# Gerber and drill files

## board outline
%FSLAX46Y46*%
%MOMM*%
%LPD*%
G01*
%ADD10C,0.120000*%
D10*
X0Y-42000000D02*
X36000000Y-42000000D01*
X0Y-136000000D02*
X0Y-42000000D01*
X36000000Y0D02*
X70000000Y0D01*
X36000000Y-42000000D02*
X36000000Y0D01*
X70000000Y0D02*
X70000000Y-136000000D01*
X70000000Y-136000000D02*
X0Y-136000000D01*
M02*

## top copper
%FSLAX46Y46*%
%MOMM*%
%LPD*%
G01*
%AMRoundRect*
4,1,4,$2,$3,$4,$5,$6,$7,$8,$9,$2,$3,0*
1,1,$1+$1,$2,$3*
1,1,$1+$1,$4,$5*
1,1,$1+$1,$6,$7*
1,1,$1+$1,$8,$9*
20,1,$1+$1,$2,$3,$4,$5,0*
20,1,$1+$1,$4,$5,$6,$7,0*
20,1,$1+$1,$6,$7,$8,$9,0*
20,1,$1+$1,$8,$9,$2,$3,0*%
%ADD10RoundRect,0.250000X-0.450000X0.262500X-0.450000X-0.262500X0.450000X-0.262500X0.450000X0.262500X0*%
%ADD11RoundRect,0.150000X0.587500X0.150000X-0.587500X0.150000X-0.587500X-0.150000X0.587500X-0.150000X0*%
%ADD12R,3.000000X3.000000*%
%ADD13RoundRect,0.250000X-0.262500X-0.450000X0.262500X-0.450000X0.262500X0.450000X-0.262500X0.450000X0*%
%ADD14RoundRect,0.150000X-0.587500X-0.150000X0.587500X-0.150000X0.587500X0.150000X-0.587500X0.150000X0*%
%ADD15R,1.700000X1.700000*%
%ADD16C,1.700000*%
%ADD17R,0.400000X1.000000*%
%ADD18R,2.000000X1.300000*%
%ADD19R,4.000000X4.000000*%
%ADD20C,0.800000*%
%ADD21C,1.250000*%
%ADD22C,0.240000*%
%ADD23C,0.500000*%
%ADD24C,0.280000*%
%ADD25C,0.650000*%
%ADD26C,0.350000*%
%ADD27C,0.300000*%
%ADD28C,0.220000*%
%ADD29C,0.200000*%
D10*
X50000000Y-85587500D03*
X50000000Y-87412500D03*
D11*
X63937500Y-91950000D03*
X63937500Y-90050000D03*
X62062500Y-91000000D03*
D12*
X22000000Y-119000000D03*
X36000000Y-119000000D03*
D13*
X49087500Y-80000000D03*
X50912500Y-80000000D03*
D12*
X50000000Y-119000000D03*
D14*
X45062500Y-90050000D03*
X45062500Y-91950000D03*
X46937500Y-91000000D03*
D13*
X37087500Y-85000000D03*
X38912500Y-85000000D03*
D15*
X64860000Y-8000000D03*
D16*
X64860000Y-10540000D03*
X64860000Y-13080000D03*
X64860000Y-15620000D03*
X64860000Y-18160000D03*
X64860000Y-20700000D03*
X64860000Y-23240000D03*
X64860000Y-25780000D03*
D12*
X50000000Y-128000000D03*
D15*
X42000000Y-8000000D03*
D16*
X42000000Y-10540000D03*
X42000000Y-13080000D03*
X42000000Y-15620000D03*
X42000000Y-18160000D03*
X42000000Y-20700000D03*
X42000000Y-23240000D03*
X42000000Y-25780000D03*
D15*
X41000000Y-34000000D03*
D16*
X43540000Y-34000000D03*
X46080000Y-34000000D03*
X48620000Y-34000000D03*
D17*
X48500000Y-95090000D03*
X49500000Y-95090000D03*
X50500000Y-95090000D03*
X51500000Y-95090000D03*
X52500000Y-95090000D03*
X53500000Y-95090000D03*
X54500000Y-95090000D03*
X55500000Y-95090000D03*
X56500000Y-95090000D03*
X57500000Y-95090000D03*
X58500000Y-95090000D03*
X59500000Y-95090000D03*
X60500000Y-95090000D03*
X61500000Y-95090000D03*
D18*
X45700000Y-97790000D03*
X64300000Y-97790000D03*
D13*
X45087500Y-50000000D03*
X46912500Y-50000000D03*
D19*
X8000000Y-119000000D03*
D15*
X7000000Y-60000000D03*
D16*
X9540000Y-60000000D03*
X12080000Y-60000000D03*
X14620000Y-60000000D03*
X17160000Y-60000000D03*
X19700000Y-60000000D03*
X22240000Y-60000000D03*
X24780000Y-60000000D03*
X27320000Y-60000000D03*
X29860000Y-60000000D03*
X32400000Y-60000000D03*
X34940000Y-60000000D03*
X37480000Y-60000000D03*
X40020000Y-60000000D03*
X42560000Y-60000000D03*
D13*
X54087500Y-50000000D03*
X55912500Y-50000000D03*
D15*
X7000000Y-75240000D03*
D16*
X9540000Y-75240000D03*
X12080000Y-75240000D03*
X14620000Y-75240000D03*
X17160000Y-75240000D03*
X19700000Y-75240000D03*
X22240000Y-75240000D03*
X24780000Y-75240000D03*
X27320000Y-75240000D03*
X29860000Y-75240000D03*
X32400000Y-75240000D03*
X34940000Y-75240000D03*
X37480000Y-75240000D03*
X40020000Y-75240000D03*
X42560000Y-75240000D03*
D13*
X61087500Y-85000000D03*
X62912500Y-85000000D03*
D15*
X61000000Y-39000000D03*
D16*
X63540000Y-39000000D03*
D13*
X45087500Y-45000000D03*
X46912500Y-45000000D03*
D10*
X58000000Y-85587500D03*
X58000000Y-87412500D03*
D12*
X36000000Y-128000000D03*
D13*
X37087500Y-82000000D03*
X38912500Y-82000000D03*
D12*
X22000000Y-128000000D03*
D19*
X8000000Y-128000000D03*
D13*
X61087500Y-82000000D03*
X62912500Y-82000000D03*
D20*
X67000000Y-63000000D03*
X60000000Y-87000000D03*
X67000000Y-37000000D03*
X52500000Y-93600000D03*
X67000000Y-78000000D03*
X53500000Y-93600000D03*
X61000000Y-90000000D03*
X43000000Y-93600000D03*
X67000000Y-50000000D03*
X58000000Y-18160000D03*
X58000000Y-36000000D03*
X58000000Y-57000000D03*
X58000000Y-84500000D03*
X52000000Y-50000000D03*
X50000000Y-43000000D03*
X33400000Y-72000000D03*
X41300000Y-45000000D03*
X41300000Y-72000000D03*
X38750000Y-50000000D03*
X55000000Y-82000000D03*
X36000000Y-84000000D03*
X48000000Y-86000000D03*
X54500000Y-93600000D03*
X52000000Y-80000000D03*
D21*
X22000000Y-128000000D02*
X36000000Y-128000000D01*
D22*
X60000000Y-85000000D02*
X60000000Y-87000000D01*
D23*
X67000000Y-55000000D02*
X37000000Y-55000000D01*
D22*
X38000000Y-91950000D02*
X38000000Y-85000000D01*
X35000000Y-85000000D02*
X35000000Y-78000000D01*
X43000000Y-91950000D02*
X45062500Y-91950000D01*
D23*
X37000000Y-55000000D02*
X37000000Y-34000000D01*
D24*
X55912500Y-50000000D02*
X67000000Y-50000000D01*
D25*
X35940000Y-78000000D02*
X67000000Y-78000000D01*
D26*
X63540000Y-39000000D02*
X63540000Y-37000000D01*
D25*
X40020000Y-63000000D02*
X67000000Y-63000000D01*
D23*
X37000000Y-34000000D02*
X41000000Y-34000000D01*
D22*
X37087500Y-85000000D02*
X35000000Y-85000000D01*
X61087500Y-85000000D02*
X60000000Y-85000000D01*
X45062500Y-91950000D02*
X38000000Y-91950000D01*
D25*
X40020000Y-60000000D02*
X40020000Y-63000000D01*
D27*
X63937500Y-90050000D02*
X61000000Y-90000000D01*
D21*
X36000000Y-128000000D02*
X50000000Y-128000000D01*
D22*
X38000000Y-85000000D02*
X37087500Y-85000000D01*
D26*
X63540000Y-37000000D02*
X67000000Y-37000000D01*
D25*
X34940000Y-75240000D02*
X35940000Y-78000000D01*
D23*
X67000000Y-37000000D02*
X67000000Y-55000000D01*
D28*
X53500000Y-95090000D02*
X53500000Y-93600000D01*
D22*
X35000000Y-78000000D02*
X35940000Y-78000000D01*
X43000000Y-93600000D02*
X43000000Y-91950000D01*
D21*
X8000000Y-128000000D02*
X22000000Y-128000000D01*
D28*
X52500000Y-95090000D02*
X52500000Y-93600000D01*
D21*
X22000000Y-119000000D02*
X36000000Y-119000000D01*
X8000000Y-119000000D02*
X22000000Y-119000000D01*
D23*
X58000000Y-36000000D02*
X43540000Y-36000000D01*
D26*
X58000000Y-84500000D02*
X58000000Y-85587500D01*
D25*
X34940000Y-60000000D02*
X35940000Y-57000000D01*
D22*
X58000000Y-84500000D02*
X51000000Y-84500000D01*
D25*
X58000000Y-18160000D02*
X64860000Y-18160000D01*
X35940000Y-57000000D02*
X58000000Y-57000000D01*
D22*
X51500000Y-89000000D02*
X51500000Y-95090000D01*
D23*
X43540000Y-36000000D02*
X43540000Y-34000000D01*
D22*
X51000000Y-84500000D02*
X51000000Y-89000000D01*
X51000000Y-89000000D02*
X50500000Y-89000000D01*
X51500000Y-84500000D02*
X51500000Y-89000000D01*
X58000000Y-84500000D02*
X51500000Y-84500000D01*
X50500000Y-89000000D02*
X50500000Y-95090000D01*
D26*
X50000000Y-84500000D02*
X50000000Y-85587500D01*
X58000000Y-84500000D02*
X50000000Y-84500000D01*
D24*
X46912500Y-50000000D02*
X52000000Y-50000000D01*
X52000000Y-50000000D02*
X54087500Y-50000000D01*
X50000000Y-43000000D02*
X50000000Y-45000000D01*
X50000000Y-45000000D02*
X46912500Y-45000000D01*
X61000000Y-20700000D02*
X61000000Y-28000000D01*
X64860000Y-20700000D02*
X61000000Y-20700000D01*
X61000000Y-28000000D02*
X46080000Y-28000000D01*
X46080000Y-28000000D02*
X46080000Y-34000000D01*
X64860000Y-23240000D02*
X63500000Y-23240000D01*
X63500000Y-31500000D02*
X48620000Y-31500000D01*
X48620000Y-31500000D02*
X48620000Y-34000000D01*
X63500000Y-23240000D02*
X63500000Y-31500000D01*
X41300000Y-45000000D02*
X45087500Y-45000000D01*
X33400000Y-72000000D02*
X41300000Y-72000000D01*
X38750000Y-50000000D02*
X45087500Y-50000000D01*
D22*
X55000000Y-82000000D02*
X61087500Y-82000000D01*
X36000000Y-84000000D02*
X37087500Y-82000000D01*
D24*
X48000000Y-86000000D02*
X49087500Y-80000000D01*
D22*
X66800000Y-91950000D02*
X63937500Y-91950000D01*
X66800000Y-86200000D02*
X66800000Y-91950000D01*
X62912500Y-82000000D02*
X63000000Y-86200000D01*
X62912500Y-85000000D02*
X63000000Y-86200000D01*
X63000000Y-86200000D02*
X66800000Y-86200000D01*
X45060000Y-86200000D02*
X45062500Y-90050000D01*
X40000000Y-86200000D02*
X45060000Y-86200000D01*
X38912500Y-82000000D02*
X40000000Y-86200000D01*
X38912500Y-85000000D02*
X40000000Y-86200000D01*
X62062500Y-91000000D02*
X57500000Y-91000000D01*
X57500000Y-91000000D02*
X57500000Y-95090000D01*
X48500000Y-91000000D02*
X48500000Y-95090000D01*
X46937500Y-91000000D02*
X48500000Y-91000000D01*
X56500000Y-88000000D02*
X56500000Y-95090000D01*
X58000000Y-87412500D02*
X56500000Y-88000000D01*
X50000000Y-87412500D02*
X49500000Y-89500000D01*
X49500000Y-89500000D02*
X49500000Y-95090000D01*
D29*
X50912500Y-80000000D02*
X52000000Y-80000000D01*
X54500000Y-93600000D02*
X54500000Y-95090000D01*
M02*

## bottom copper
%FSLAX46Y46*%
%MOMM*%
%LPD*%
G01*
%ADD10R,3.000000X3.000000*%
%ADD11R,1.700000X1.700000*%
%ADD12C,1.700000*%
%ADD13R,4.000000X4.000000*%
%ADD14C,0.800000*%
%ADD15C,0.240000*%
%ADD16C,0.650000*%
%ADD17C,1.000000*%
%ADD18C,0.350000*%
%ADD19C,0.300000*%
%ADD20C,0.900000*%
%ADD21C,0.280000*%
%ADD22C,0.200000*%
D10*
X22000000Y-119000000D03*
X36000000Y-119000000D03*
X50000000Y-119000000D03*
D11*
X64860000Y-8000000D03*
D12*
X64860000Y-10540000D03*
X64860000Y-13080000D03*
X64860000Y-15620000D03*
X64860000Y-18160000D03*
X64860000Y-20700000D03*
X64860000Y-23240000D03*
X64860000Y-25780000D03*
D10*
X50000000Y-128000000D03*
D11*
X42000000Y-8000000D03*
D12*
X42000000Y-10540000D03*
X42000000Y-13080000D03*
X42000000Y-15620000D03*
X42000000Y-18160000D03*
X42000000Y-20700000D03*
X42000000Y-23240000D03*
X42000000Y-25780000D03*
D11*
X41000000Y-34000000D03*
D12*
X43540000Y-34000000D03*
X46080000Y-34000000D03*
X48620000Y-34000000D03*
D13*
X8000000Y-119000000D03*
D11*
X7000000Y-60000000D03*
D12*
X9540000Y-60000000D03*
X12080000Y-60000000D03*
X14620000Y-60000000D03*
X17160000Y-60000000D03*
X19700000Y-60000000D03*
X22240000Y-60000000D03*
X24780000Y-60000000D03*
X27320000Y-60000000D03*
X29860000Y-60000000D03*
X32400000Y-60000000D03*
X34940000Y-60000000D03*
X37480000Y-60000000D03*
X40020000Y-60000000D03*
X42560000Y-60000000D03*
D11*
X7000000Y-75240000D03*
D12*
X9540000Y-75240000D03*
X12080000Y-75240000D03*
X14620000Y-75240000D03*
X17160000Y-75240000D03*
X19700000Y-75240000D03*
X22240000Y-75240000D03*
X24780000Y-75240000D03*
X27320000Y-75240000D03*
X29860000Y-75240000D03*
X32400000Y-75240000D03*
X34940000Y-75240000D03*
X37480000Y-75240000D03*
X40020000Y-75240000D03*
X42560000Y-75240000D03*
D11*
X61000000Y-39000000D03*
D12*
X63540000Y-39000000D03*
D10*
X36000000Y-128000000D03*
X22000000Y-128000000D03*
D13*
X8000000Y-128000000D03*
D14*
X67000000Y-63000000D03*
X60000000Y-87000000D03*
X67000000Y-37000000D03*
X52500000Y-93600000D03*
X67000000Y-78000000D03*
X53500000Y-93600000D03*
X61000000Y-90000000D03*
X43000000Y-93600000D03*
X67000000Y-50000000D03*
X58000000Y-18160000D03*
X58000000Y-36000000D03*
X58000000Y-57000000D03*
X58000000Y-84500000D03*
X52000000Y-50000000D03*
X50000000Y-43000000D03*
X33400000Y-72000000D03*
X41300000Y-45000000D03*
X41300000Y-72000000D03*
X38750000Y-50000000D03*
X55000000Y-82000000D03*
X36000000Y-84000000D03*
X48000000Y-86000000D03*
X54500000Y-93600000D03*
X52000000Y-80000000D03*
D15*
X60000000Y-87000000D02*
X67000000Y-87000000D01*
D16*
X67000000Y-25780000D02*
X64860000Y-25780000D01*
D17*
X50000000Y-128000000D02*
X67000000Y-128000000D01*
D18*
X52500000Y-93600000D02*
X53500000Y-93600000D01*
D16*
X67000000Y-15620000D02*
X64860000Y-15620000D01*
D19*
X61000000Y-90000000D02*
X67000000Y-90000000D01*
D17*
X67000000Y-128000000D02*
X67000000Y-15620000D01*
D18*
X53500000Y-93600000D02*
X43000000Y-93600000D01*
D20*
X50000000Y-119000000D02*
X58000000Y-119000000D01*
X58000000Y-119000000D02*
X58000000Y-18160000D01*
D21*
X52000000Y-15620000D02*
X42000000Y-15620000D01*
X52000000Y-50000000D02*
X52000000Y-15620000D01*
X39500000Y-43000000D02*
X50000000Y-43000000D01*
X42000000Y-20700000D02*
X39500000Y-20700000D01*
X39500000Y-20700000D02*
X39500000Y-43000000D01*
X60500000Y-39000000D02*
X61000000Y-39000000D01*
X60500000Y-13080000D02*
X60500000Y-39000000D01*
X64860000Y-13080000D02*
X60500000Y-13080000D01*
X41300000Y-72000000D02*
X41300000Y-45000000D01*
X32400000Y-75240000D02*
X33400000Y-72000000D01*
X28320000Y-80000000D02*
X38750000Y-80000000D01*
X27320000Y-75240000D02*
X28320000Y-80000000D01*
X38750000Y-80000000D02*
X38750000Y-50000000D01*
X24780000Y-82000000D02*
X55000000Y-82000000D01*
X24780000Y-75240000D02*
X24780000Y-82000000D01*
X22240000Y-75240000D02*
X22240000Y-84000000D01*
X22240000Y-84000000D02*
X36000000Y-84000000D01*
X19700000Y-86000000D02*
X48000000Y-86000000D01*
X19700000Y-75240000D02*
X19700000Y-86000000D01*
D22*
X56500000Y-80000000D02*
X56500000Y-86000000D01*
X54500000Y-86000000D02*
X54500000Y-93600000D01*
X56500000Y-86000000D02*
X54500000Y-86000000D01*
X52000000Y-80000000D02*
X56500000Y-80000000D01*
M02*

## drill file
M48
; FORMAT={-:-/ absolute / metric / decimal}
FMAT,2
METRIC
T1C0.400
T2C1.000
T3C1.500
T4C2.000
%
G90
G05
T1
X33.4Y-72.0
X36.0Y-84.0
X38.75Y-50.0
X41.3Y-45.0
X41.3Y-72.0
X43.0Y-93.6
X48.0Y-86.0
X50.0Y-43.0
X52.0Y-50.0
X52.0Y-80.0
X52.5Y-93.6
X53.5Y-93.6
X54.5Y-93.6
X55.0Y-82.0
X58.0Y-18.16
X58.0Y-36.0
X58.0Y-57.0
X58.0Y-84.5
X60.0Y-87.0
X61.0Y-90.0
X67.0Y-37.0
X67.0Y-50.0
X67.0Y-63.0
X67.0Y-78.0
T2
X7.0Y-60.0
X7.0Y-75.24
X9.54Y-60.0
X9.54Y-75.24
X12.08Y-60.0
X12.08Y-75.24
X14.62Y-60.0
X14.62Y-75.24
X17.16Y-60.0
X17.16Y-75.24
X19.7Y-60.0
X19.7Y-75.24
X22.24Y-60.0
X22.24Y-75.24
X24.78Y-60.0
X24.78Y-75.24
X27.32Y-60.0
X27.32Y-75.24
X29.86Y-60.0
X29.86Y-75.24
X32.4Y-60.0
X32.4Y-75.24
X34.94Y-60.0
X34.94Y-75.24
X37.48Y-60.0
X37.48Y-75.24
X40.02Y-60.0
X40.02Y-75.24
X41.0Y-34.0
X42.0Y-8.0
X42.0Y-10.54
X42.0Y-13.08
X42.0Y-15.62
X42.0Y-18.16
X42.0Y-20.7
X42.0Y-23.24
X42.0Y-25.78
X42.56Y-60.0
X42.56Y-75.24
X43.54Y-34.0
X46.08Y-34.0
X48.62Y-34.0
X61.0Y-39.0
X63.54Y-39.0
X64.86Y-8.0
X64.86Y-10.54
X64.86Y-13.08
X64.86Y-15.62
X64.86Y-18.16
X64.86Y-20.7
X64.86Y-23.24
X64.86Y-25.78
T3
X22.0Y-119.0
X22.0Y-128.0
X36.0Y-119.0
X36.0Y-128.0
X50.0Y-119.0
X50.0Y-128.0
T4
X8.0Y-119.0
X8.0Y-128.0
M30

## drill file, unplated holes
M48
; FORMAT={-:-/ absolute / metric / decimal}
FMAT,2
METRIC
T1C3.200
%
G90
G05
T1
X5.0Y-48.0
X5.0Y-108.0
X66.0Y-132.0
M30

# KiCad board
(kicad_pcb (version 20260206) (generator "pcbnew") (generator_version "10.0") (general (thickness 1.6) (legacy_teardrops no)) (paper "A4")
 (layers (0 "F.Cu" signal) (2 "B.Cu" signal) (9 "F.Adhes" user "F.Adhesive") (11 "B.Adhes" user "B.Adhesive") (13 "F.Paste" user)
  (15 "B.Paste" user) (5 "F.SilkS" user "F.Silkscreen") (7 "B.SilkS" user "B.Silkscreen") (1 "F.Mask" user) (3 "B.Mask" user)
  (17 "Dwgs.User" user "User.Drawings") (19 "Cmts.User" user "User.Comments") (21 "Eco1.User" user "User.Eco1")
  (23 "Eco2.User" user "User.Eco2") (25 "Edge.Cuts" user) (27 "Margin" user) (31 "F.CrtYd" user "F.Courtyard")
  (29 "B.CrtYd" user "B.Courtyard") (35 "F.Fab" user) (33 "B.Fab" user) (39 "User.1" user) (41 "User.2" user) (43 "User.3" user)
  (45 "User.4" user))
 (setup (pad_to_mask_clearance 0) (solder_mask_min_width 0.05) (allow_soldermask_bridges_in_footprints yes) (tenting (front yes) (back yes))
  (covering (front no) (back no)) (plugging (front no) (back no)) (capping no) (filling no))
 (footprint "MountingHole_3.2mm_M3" (layer "F.Cu") (at 5 48)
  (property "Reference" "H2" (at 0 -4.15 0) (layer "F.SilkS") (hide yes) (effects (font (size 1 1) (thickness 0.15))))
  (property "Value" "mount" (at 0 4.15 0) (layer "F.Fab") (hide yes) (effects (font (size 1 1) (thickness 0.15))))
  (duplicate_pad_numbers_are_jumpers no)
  (pad "" np_thru_hole circle (at 0 0) (size 3.2 3.2) (drill 3.2) (layers "*.Cu" "*.Mask")))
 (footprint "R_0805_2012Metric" (layer "F.Cu") (at 50 86.5 -90)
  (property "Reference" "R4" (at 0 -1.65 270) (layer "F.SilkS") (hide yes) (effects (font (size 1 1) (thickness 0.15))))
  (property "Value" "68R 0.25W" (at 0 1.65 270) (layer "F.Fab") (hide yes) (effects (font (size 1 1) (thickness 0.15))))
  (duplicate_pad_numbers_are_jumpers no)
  (pad "1" smd roundrect (at -0.9125 0 270) (size 1.025 1.4) (layers "F.Cu" "F.Mask" "F.Paste") (roundrect_rratio 0.243902) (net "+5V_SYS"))
  (pad "2" smd roundrect (at 0.9125 0 270) (size 1.025 1.4) (layers "F.Cu" "F.Mask" "F.Paste") (roundrect_rratio 0.243902) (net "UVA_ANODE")))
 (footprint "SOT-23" (layer "F.Cu") (at 63 91 180)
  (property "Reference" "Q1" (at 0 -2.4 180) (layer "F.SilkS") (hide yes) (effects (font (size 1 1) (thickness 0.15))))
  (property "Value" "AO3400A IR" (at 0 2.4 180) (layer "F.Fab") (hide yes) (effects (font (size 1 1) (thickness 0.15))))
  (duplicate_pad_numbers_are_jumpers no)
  (pad "1" smd roundrect (at -0.9375 -0.95 180) (size 1.475 0.6) (layers "F.Cu" "F.Mask" "F.Paste") (roundrect_rratio 0.25) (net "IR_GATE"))
  (pad "2" smd roundrect (at -0.9375 0.95 180) (size 1.475 0.6) (layers "F.Cu" "F.Mask" "F.Paste") (roundrect_rratio 0.25) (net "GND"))
  (pad "3" smd roundrect (at 0.9375 0 180) (size 1.475 0.6) (layers "F.Cu" "F.Mask" "F.Paste") (roundrect_rratio 0.25) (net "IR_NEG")))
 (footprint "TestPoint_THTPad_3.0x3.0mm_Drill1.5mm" (layer "F.Cu") (at 22 119)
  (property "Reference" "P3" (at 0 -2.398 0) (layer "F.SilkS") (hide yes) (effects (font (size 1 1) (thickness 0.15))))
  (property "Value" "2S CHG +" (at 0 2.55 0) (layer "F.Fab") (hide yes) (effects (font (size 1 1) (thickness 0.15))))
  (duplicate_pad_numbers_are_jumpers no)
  (pad "1" thru_hole rect (at 0 0) (size 3 3) (drill 1.5) (layers "*.Cu" "*.Mask") (remove_unused_layers no) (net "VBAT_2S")))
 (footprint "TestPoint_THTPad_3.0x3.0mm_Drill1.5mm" (layer "F.Cu") (at 36 119)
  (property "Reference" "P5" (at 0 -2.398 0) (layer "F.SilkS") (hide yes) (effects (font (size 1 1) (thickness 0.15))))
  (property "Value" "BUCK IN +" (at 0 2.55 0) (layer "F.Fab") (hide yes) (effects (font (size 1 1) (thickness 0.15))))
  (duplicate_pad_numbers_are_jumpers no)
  (pad "1" thru_hole rect (at 0 0) (size 3 3) (drill 1.5) (layers "*.Cu" "*.Mask") (remove_unused_layers no) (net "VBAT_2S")))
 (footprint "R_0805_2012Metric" (layer "F.Cu") (at 50 80)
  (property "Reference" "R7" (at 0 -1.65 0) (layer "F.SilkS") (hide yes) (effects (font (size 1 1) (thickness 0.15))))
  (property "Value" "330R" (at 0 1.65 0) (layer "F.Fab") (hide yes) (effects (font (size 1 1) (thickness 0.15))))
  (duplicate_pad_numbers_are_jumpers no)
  (pad "1" smd roundrect (at -0.9125 0) (size 1.025 1.4) (layers "F.Cu" "F.Mask" "F.Paste") (roundrect_rratio 0.243902)
   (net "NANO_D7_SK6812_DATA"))
  (pad "2" smd roundrect (at 0.9125 0) (size 1.025 1.4) (layers "F.Cu" "F.Mask" "F.Paste") (roundrect_rratio 0.243902) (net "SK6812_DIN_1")))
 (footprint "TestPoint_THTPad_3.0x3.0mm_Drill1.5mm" (layer "F.Cu") (at 50 119)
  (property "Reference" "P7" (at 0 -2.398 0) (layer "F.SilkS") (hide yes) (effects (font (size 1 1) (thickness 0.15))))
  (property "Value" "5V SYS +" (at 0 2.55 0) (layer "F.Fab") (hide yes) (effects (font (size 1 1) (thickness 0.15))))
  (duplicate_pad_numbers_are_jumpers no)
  (pad "1" thru_hole rect (at 0 0) (size 3 3) (drill 1.5) (layers "*.Cu" "*.Mask") (remove_unused_layers no) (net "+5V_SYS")))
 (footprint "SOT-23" (layer "F.Cu") (at 46 91)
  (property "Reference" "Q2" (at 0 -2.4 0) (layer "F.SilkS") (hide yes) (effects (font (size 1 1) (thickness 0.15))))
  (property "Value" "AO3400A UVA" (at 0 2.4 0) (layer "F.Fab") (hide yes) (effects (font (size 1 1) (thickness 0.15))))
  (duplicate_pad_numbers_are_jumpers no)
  (pad "1" smd roundrect (at -0.9375 -0.95) (size 1.475 0.6) (layers "F.Cu" "F.Mask" "F.Paste") (roundrect_rratio 0.25) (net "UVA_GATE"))
  (pad "2" smd roundrect (at -0.9375 0.95) (size 1.475 0.6) (layers "F.Cu" "F.Mask" "F.Paste") (roundrect_rratio 0.25) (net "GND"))
  (pad "3" smd roundrect (at 0.9375 0) (size 1.475 0.6) (layers "F.Cu" "F.Mask" "F.Paste") (roundrect_rratio 0.25) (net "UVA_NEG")))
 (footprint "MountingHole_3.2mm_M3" (layer "F.Cu") (at 66 132)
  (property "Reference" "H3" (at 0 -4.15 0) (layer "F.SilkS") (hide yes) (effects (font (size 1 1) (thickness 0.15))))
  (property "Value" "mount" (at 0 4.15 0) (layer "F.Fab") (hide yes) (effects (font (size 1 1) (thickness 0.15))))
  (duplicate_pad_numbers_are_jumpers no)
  (pad "" np_thru_hole circle (at 0 0) (size 3.2 3.2) (drill 3.2) (layers "*.Cu" "*.Mask")))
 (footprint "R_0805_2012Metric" (layer "F.Cu") (at 38 85)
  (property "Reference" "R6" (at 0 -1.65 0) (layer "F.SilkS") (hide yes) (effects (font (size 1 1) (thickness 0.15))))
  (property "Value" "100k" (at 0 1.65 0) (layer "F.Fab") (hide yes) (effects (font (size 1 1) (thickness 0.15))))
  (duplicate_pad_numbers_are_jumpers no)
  (pad "1" smd roundrect (at -0.9125 0) (size 1.025 1.4) (layers "F.Cu" "F.Mask" "F.Paste") (roundrect_rratio 0.243902) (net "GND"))
  (pad "2" smd roundrect (at 0.9125 0) (size 1.025 1.4) (layers "F.Cu" "F.Mask" "F.Paste") (roundrect_rratio 0.243902) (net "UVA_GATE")))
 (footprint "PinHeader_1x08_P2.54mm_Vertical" (layer "F.Cu") (at 64.86 8)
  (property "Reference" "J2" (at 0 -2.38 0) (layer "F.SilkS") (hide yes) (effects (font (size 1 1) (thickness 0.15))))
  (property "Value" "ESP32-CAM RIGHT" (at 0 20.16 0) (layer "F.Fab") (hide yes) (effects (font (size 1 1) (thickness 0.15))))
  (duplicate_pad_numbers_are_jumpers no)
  (pad "1" thru_hole rect (at 0 0) (size 1.7 1.7) (drill 1) (layers "*.Cu" "*.Mask") (remove_unused_layers no))
  (pad "2" thru_hole circle (at 0 2.54) (size 1.7 1.7) (drill 1) (layers "*.Cu" "*.Mask") (remove_unused_layers no))
  (pad "3" thru_hole circle (at 0 5.08) (size 1.7 1.7) (drill 1) (layers "*.Cu" "*.Mask") (remove_unused_layers no) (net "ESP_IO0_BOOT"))
  (pad "4" thru_hole circle (at 0 7.62) (size 1.7 1.7) (drill 1) (layers "*.Cu" "*.Mask") (remove_unused_layers no) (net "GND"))
  (pad "5" thru_hole circle (at 0 10.16) (size 1.7 1.7) (drill 1) (layers "*.Cu" "*.Mask") (remove_unused_layers no) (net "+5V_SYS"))
  (pad "6" thru_hole circle (at 0 12.7) (size 1.7 1.7) (drill 1) (layers "*.Cu" "*.Mask") (remove_unused_layers no) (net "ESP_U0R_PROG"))
  (pad "7" thru_hole circle (at 0 15.24) (size 1.7 1.7) (drill 1) (layers "*.Cu" "*.Mask") (remove_unused_layers no) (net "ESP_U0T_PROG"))
  (pad "8" thru_hole circle (at 0 17.78) (size 1.7 1.7) (drill 1) (layers "*.Cu" "*.Mask") (remove_unused_layers no) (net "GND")))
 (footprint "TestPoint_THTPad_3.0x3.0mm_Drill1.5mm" (layer "F.Cu") (at 50 128)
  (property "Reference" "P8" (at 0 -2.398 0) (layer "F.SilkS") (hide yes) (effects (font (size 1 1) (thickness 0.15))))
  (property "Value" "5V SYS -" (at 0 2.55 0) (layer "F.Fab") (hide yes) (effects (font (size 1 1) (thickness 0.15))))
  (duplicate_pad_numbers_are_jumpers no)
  (pad "1" thru_hole rect (at 0 0) (size 3 3) (drill 1.5) (layers "*.Cu" "*.Mask") (remove_unused_layers no) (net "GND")))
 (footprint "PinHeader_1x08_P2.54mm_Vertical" (layer "F.Cu") (at 42 8)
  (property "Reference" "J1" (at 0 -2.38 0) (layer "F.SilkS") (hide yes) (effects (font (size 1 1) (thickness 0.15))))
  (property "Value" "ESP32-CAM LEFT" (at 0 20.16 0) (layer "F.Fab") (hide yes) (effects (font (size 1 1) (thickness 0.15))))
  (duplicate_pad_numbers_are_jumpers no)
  (pad "1" thru_hole rect (at 0 0) (size 1.7 1.7) (drill 1) (layers "*.Cu" "*.Mask") (remove_unused_layers no))
  (pad "2" thru_hole circle (at 0 2.54) (size 1.7 1.7) (drill 1) (layers "*.Cu" "*.Mask") (remove_unused_layers no))
  (pad "3" thru_hole circle (at 0 5.08) (size 1.7 1.7) (drill 1) (layers "*.Cu" "*.Mask") (remove_unused_layers no))
  (pad "4" thru_hole circle (at 0 7.62) (size 1.7 1.7) (drill 1) (layers "*.Cu" "*.Mask") (remove_unused_layers no) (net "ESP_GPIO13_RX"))
  (pad "5" thru_hole circle (at 0 10.16) (size 1.7 1.7) (drill 1) (layers "*.Cu" "*.Mask") (remove_unused_layers no))
  (pad "6" thru_hole circle (at 0 12.7) (size 1.7 1.7) (drill 1) (layers "*.Cu" "*.Mask") (remove_unused_layers no) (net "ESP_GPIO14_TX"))
  (pad "7" thru_hole circle (at 0 15.24) (size 1.7 1.7) (drill 1) (layers "*.Cu" "*.Mask") (remove_unused_layers no))
  (pad "8" thru_hole circle (at 0 17.78) (size 1.7 1.7) (drill 1) (layers "*.Cu" "*.Mask") (remove_unused_layers no)))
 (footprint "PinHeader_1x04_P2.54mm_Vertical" (layer "F.Cu") (at 41 34 90)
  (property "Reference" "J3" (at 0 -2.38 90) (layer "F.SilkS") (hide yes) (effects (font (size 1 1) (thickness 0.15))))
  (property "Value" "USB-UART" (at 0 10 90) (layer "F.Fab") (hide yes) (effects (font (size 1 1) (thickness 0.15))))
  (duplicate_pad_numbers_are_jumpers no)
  (pad "1" thru_hole rect (at 0 0 90) (size 1.7 1.7) (drill 1) (layers "*.Cu" "*.Mask") (remove_unused_layers no) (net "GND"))
  (pad "2" thru_hole circle (at 0 2.54 90) (size 1.7 1.7) (drill 1) (layers "*.Cu" "*.Mask") (remove_unused_layers no) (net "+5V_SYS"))
  (pad "3" thru_hole circle (at 0 5.08 90) (size 1.7 1.7) (drill 1) (layers "*.Cu" "*.Mask") (remove_unused_layers no) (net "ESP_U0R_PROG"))
  (pad "4" thru_hole circle (at 0 7.62 90) (size 1.7 1.7) (drill 1) (layers "*.Cu" "*.Mask") (remove_unused_layers no) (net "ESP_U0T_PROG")))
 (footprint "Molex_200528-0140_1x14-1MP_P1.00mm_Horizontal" (layer "F.Cu") (at 55 96)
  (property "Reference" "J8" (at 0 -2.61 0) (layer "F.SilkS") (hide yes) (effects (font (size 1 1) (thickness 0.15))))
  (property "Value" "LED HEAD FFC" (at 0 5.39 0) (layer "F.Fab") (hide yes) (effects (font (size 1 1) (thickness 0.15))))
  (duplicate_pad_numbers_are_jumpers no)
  (pad "1" smd rect (at -6.5 -0.91) (size 0.4 1) (layers "F.Cu" "F.Mask" "F.Paste") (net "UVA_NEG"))
  (pad "2" smd rect (at -5.5 -0.91) (size 0.4 1) (layers "F.Cu" "F.Mask" "F.Paste") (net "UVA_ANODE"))
  (pad "3" smd rect (at -4.5 -0.91) (size 0.4 1) (layers "F.Cu" "F.Mask" "F.Paste") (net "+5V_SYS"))
  (pad "4" smd rect (at -3.5 -0.91) (size 0.4 1) (layers "F.Cu" "F.Mask" "F.Paste") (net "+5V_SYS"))
  (pad "5" smd rect (at -2.5 -0.91) (size 0.4 1) (layers "F.Cu" "F.Mask" "F.Paste") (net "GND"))
  (pad "6" smd rect (at -1.5 -0.91) (size 0.4 1) (layers "F.Cu" "F.Mask" "F.Paste") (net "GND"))
  (pad "7" smd rect (at -0.5 -0.91) (size 0.4 1) (layers "F.Cu" "F.Mask" "F.Paste") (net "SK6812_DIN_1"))
  (pad "8" smd rect (at 0.5 -0.91) (size 0.4 1) (layers "F.Cu" "F.Mask" "F.Paste"))
  (pad "9" smd rect (at 1.5 -0.91) (size 0.4 1) (layers "F.Cu" "F.Mask" "F.Paste") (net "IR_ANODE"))
  (pad "10" smd rect (at 2.5 -0.91) (size 0.4 1) (layers "F.Cu" "F.Mask" "F.Paste") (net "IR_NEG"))
  (pad "11" smd rect (at 3.5 -0.91) (size 0.4 1) (layers "F.Cu" "F.Mask" "F.Paste"))
  (pad "12" smd rect (at 4.5 -0.91) (size 0.4 1) (layers "F.Cu" "F.Mask" "F.Paste"))
  (pad "13" smd rect (at 5.5 -0.91) (size 0.4 1) (layers "F.Cu" "F.Mask" "F.Paste"))
  (pad "14" smd rect (at 6.5 -0.91) (size 0.4 1) (layers "F.Cu" "F.Mask" "F.Paste"))
  (pad "MP" smd rect (at -9.3 1.79) (size 2 1.3) (layers "F.Cu" "F.Mask" "F.Paste"))
  (pad "MP" smd rect (at 9.3 1.79) (size 2 1.3) (layers "F.Cu" "F.Mask" "F.Paste")))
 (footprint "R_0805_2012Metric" (layer "F.Cu") (at 46 50)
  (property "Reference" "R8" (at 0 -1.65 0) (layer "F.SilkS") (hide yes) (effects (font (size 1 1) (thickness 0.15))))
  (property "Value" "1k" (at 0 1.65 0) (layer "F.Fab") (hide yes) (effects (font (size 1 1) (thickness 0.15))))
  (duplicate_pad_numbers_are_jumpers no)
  (pad "1" smd roundrect (at -0.9125 0) (size 1.025 1.4) (layers "F.Cu" "F.Mask" "F.Paste") (roundrect_rratio 0.243902) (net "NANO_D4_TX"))
  (pad "2" smd roundrect (at 0.9125 0) (size 1.025 1.4) (layers "F.Cu" "F.Mask" "F.Paste") (roundrect_rratio 0.243902) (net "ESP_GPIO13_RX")))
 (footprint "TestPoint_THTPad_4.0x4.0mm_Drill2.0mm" (layer "F.Cu") (at 8 119)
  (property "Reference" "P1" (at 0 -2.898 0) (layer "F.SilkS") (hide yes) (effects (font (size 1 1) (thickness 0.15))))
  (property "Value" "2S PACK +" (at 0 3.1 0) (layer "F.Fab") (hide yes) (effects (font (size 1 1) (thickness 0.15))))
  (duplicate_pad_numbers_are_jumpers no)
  (pad "1" thru_hole rect (at 0 0) (size 4 4) (drill 2) (layers "*.Cu" "*.Mask") (remove_unused_layers no) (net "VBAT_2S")))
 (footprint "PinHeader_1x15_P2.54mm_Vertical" (layer "F.Cu") (at 7 60 90)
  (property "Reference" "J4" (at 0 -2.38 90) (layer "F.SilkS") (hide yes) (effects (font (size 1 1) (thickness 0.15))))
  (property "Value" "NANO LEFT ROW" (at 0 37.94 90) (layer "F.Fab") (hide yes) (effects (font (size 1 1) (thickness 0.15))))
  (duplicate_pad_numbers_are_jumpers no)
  (pad "1" thru_hole rect (at 0 0 90) (size 1.7 1.7) (drill 1) (layers "*.Cu" "*.Mask") (remove_unused_layers no))
  (pad "2" thru_hole circle (at 0 2.54 90) (size 1.7 1.7) (drill 1) (layers "*.Cu" "*.Mask") (remove_unused_layers no))
  (pad "3" thru_hole circle (at 0 5.08 90) (size 1.7 1.7) (drill 1) (layers "*.Cu" "*.Mask") (remove_unused_layers no))
  (pad "4" thru_hole circle (at 0 7.62 90) (size 1.7 1.7) (drill 1) (layers "*.Cu" "*.Mask") (remove_unused_layers no))
  (pad "5" thru_hole circle (at 0 10.16 90) (size 1.7 1.7) (drill 1) (layers "*.Cu" "*.Mask") (remove_unused_layers no))
  (pad "6" thru_hole circle (at 0 12.7 90) (size 1.7 1.7) (drill 1) (layers "*.Cu" "*.Mask") (remove_unused_layers no))
  (pad "7" thru_hole circle (at 0 15.24 90) (size 1.7 1.7) (drill 1) (layers "*.Cu" "*.Mask") (remove_unused_layers no))
  (pad "8" thru_hole circle (at 0 17.78 90) (size 1.7 1.7) (drill 1) (layers "*.Cu" "*.Mask") (remove_unused_layers no))
  (pad "9" thru_hole circle (at 0 20.32 90) (size 1.7 1.7) (drill 1) (layers "*.Cu" "*.Mask") (remove_unused_layers no))
  (pad "10" thru_hole circle (at 0 22.86 90) (size 1.7 1.7) (drill 1) (layers "*.Cu" "*.Mask") (remove_unused_layers no))
  (pad "11" thru_hole circle (at 0 25.4 90) (size 1.7 1.7) (drill 1) (layers "*.Cu" "*.Mask") (remove_unused_layers no))
  (pad "12" thru_hole circle (at 0 27.94 90) (size 1.7 1.7) (drill 1) (layers "*.Cu" "*.Mask") (remove_unused_layers no) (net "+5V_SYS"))
  (pad "13" thru_hole circle (at 0 30.48 90) (size 1.7 1.7) (drill 1) (layers "*.Cu" "*.Mask") (remove_unused_layers no))
  (pad "14" thru_hole circle (at 0 33.02 90) (size 1.7 1.7) (drill 1) (layers "*.Cu" "*.Mask") (remove_unused_layers no) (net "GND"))
  (pad "15" thru_hole circle (at 0 35.56 90) (size 1.7 1.7) (drill 1) (layers "*.Cu" "*.Mask") (remove_unused_layers no)))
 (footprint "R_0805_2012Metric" (layer "F.Cu") (at 55 50)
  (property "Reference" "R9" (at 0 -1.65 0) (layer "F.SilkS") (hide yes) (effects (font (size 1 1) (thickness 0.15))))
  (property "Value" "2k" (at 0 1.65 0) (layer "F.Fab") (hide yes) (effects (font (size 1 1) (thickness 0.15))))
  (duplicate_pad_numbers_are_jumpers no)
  (pad "1" smd roundrect (at -0.9125 0) (size 1.025 1.4) (layers "F.Cu" "F.Mask" "F.Paste") (roundrect_rratio 0.243902)
   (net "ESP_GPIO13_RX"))
  (pad "2" smd roundrect (at 0.9125 0) (size 1.025 1.4) (layers "F.Cu" "F.Mask" "F.Paste") (roundrect_rratio 0.243902) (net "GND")))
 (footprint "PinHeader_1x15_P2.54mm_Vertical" (layer "F.Cu") (at 7 75.24 90)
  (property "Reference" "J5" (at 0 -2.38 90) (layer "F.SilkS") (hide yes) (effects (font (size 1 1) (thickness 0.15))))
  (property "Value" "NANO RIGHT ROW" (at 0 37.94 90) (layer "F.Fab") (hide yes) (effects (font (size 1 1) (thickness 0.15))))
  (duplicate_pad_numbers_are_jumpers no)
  (pad "1" thru_hole rect (at 0 0 90) (size 1.7 1.7) (drill 1) (layers "*.Cu" "*.Mask") (remove_unused_layers no))
  (pad "2" thru_hole circle (at 0 2.54 90) (size 1.7 1.7) (drill 1) (layers "*.Cu" "*.Mask") (remove_unused_layers no))
  (pad "3" thru_hole circle (at 0 5.08 90) (size 1.7 1.7) (drill 1) (layers "*.Cu" "*.Mask") (remove_unused_layers no))
  (pad "4" thru_hole circle (at 0 7.62 90) (size 1.7 1.7) (drill 1) (layers "*.Cu" "*.Mask") (remove_unused_layers no))
  (pad "5" thru_hole circle (at 0 10.16 90) (size 1.7 1.7) (drill 1) (layers "*.Cu" "*.Mask") (remove_unused_layers no)
   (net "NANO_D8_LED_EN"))
  (pad "6" thru_hole circle (at 0 12.7 90) (size 1.7 1.7) (drill 1) (layers "*.Cu" "*.Mask") (remove_unused_layers no)
   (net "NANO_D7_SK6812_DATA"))
  (pad "7" thru_hole circle (at 0 15.24 90) (size 1.7 1.7) (drill 1) (layers "*.Cu" "*.Mask") (remove_unused_layers no)
   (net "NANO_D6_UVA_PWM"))
  (pad "8" thru_hole circle (at 0 17.78 90) (size 1.7 1.7) (drill 1) (layers "*.Cu" "*.Mask") (remove_unused_layers no)
   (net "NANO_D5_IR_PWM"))
  (pad "9" thru_hole circle (at 0 20.32 90) (size 1.7 1.7) (drill 1) (layers "*.Cu" "*.Mask") (remove_unused_layers no) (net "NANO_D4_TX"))
  (pad "10" thru_hole circle (at 0 22.86 90) (size 1.7 1.7) (drill 1) (layers "*.Cu" "*.Mask") (remove_unused_layers no))
  (pad "11" thru_hole circle (at 0 25.4 90) (size 1.7 1.7) (drill 1) (layers "*.Cu" "*.Mask") (remove_unused_layers no) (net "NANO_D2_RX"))
  (pad "12" thru_hole circle (at 0 27.94 90) (size 1.7 1.7) (drill 1) (layers "*.Cu" "*.Mask") (remove_unused_layers no) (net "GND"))
  (pad "13" thru_hole circle (at 0 30.48 90) (size 1.7 1.7) (drill 1) (layers "*.Cu" "*.Mask") (remove_unused_layers no))
  (pad "14" thru_hole circle (at 0 33.02 90) (size 1.7 1.7) (drill 1) (layers "*.Cu" "*.Mask") (remove_unused_layers no))
  (pad "15" thru_hole circle (at 0 35.56 90) (size 1.7 1.7) (drill 1) (layers "*.Cu" "*.Mask") (remove_unused_layers no)))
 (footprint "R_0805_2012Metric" (layer "F.Cu") (at 62 85)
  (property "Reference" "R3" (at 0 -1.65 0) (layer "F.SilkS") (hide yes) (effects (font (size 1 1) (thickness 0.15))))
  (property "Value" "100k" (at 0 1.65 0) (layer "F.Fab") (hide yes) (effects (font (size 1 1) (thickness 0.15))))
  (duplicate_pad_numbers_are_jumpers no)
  (pad "1" smd roundrect (at -0.9125 0) (size 1.025 1.4) (layers "F.Cu" "F.Mask" "F.Paste") (roundrect_rratio 0.243902) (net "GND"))
  (pad "2" smd roundrect (at 0.9125 0) (size 1.025 1.4) (layers "F.Cu" "F.Mask" "F.Paste") (roundrect_rratio 0.243902) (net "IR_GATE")))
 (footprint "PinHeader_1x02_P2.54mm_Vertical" (layer "F.Cu") (at 61 39 90)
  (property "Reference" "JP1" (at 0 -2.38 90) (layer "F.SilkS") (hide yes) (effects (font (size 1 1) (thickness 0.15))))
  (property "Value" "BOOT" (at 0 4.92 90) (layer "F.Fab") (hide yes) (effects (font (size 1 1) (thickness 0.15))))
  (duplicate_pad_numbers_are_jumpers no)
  (pad "1" thru_hole rect (at 0 0 90) (size 1.7 1.7) (drill 1) (layers "*.Cu" "*.Mask") (remove_unused_layers no) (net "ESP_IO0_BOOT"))
  (pad "2" thru_hole circle (at 0 2.54 90) (size 1.7 1.7) (drill 1) (layers "*.Cu" "*.Mask") (remove_unused_layers no) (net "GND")))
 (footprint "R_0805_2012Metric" (layer "F.Cu") (at 46 45)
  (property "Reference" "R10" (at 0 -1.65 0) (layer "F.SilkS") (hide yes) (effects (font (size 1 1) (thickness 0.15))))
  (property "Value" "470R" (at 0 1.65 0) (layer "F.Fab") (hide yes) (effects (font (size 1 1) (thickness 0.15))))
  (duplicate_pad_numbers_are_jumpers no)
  (pad "1" smd roundrect (at -0.9125 0) (size 1.025 1.4) (layers "F.Cu" "F.Mask" "F.Paste") (roundrect_rratio 0.243902) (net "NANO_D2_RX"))
  (pad "2" smd roundrect (at 0.9125 0) (size 1.025 1.4) (layers "F.Cu" "F.Mask" "F.Paste") (roundrect_rratio 0.243902) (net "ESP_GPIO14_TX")))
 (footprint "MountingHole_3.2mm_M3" (layer "F.Cu") (at 5 108)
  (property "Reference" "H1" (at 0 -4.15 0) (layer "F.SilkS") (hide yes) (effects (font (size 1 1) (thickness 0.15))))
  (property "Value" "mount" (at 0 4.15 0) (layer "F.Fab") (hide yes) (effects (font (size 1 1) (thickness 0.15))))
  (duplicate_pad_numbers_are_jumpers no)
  (pad "" np_thru_hole circle (at 0 0) (size 3.2 3.2) (drill 3.2) (layers "*.Cu" "*.Mask")))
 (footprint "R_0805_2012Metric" (layer "F.Cu") (at 58 86.5 -90)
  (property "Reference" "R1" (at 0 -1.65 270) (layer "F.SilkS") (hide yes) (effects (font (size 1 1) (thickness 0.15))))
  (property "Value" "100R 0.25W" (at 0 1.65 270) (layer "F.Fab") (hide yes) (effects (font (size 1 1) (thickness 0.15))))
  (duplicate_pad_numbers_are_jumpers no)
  (pad "1" smd roundrect (at -0.9125 0 270) (size 1.025 1.4) (layers "F.Cu" "F.Mask" "F.Paste") (roundrect_rratio 0.243902) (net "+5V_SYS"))
  (pad "2" smd roundrect (at 0.9125 0 270) (size 1.025 1.4) (layers "F.Cu" "F.Mask" "F.Paste") (roundrect_rratio 0.243902) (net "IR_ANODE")))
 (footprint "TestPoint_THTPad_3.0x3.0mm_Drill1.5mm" (layer "F.Cu") (at 36 128)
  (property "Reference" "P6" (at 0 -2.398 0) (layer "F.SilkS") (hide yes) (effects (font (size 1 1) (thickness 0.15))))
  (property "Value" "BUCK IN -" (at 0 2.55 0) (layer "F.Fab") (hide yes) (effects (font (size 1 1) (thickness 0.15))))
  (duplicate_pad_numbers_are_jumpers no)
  (pad "1" thru_hole rect (at 0 0) (size 3 3) (drill 1.5) (layers "*.Cu" "*.Mask") (remove_unused_layers no) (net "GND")))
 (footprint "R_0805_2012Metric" (layer "F.Cu") (at 38 82)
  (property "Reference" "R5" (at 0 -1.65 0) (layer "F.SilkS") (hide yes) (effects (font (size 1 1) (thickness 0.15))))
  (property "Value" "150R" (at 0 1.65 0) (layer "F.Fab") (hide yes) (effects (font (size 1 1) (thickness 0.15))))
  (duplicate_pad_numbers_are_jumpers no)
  (pad "1" smd roundrect (at -0.9125 0) (size 1.025 1.4) (layers "F.Cu" "F.Mask" "F.Paste") (roundrect_rratio 0.243902)
   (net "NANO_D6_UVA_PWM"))
  (pad "2" smd roundrect (at 0.9125 0) (size 1.025 1.4) (layers "F.Cu" "F.Mask" "F.Paste") (roundrect_rratio 0.243902) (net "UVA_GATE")))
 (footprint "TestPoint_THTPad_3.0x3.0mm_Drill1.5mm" (layer "F.Cu") (at 22 128)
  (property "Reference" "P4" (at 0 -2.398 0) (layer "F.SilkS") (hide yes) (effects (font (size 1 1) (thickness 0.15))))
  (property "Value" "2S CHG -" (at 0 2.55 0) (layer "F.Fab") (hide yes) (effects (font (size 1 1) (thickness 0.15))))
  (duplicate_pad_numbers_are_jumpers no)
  (pad "1" thru_hole rect (at 0 0) (size 3 3) (drill 1.5) (layers "*.Cu" "*.Mask") (remove_unused_layers no) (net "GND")))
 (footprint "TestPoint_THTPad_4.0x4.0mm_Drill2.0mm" (layer "F.Cu") (at 8 128)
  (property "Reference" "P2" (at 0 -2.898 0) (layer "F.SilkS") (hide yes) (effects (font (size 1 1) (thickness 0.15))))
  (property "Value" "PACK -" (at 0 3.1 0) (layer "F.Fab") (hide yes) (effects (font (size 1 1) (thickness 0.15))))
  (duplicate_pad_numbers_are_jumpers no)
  (pad "1" thru_hole rect (at 0 0) (size 4 4) (drill 2) (layers "*.Cu" "*.Mask") (remove_unused_layers no) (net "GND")))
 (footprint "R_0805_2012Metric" (layer "F.Cu") (at 62 82)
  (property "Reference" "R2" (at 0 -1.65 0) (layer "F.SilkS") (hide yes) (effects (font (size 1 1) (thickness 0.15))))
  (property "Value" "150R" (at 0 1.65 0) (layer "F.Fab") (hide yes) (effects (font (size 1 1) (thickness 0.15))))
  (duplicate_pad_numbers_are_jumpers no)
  (pad "1" smd roundrect (at -0.9125 0) (size 1.025 1.4) (layers "F.Cu" "F.Mask" "F.Paste") (roundrect_rratio 0.243902)
   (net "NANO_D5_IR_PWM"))
  (pad "2" smd roundrect (at 0.9125 0) (size 1.025 1.4) (layers "F.Cu" "F.Mask" "F.Paste") (roundrect_rratio 0.243902) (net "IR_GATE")))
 (gr_line (start 0 42) (end 36 42) (stroke (width 0.12) (type default)) (layer "Edge.Cuts"))
 (gr_line (start 0 136) (end 0 42) (stroke (width 0.12) (type default)) (layer "Edge.Cuts"))
 (gr_line (start 36 0) (end 70 0) (stroke (width 0.12) (type default)) (layer "Edge.Cuts"))
 (gr_line (start 36 42) (end 36 0) (stroke (width 0.12) (type default)) (layer "Edge.Cuts"))
 (gr_line (start 70 0) (end 70 136) (stroke (width 0.12) (type default)) (layer "Edge.Cuts"))
 (gr_line (start 70 136) (end 0 136) (stroke (width 0.12) (type default)) (layer "Edge.Cuts"))
 (segment (start 22 128) (end 36 128) (width 1.25) (layer "F.Cu") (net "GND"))
 (segment (start 60 85) (end 60 87) (width 0.24) (layer "F.Cu") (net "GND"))
 (segment (start 67 55) (end 37 55) (width 0.5) (layer "F.Cu") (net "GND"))
 (segment (start 38 91.95) (end 38 85) (width 0.24) (layer "F.Cu") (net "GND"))
 (segment (start 35 85) (end 35 78) (width 0.24) (layer "F.Cu") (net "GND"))
 (segment (start 43 91.95) (end 45.0625 91.95) (width 0.24) (layer "F.Cu") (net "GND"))
 (segment (start 37 55) (end 37 34) (width 0.5) (layer "F.Cu") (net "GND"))
 (segment (start 55.9125 50) (end 67 50) (width 0.28) (layer "F.Cu") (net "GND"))
 (segment (start 35.94 78) (end 67 78) (width 0.65) (layer "F.Cu") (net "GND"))
 (segment (start 63.54 39) (end 63.54 37) (width 0.35) (layer "F.Cu") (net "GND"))
 (segment (start 40.02 63) (end 67 63) (width 0.65) (layer "F.Cu") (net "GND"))
 (segment (start 37 34) (end 41 34) (width 0.5) (layer "F.Cu") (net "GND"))
 (segment (start 37.0875 85) (end 35 85) (width 0.24) (layer "F.Cu") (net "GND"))
 (segment (start 61.0875 85) (end 60 85) (width 0.24) (layer "F.Cu") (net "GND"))
 (segment (start 45.0625 91.95) (end 38 91.95) (width 0.24) (layer "F.Cu") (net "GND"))
 (segment (start 40.02 60) (end 40.02 63) (width 0.65) (layer "F.Cu") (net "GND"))
 (segment (start 63.9375 90.05) (end 61 90) (width 0.3) (layer "F.Cu") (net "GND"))
 (segment (start 36 128) (end 50 128) (width 1.25) (layer "F.Cu") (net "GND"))
 (segment (start 38 85) (end 37.0875 85) (width 0.24) (layer "F.Cu") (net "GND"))
 (segment (start 63.54 37) (end 67 37) (width 0.35) (layer "F.Cu") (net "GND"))
 (segment (start 34.94 75.24) (end 35.94 78) (width 0.65) (layer "F.Cu") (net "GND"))
 (segment (start 67 37) (end 67 55) (width 0.5) (layer "F.Cu") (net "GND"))
 (segment (start 53.5 95.09) (end 53.5 93.6) (width 0.22) (layer "F.Cu") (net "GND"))
 (segment (start 35 78) (end 35.94 78) (width 0.24) (layer "F.Cu") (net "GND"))
 (segment (start 43 93.6) (end 43 91.95) (width 0.24) (layer "F.Cu") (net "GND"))
 (segment (start 8 128) (end 22 128) (width 1.25) (layer "F.Cu") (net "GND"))
 (segment (start 52.5 95.09) (end 52.5 93.6) (width 0.22) (layer "F.Cu") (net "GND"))
 (via (at 67 63) (size 0.8) (drill 0.4) (layers "F.Cu" "B.Cu") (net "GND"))
 (via (at 60 87) (size 0.8) (drill 0.4) (layers "F.Cu" "B.Cu") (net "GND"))
 (via (at 67 37) (size 0.8) (drill 0.4) (layers "F.Cu" "B.Cu") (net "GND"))
 (via (at 52.5 93.6) (size 0.8) (drill 0.4) (layers "F.Cu" "B.Cu") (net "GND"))
 (via (at 67 78) (size 0.8) (drill 0.4) (layers "F.Cu" "B.Cu") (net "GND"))
 (via (at 53.5 93.6) (size 0.8) (drill 0.4) (layers "F.Cu" "B.Cu") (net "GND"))
 (via (at 61 90) (size 0.8) (drill 0.4) (layers "F.Cu" "B.Cu") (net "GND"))
 (via (at 43 93.6) (size 0.8) (drill 0.4) (layers "F.Cu" "B.Cu") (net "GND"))
 (via (at 67 50) (size 0.8) (drill 0.4) (layers "F.Cu" "B.Cu") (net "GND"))
 (segment (start 60 87) (end 67 87) (width 0.24) (layer "B.Cu") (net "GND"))
 (segment (start 67 25.78) (end 64.86 25.78) (width 0.65) (layer "B.Cu") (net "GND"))
 (segment (start 50 128) (end 67 128) (width 1) (layer "B.Cu") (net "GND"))
 (segment (start 52.5 93.6) (end 53.5 93.6) (width 0.35) (layer "B.Cu") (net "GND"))
 (segment (start 67 15.62) (end 64.86 15.62) (width 0.65) (layer "B.Cu") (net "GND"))
 (segment (start 61 90) (end 67 90) (width 0.3) (layer "B.Cu") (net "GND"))
 (segment (start 67 128) (end 67 15.62) (width 1) (layer "B.Cu") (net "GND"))
 (segment (start 53.5 93.6) (end 43 93.6) (width 0.35) (layer "B.Cu") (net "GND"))
 (segment (start 22 119) (end 36 119) (width 1.25) (layer "F.Cu") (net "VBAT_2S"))
 (segment (start 8 119) (end 22 119) (width 1.25) (layer "F.Cu") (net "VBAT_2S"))
 (segment (start 58 36) (end 43.54 36) (width 0.5) (layer "F.Cu") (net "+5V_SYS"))
 (segment (start 58 84.5) (end 58 85.5875) (width 0.35) (layer "F.Cu") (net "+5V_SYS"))
 (segment (start 34.94 60) (end 35.94 57) (width 0.65) (layer "F.Cu") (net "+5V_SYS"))
 (segment (start 58 84.5) (end 51 84.5) (width 0.24) (layer "F.Cu") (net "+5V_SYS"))
 (segment (start 58 18.16) (end 64.86 18.16) (width 0.65) (layer "F.Cu") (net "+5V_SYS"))
 (segment (start 35.94 57) (end 58 57) (width 0.65) (layer "F.Cu") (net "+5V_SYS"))
 (segment (start 51.5 89) (end 51.5 95.09) (width 0.24) (layer "F.Cu") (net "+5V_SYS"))
 (segment (start 43.54 36) (end 43.54 34) (width 0.5) (layer "F.Cu") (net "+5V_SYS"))
 (segment (start 51 84.5) (end 51 89) (width 0.24) (layer "F.Cu") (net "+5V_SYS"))
 (segment (start 51 89) (end 50.5 89) (width 0.24) (layer "F.Cu") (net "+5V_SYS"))
 (segment (start 51.5 84.5) (end 51.5 89) (width 0.24) (layer "F.Cu") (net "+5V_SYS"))
 (segment (start 58 84.5) (end 51.5 84.5) (width 0.24) (layer "F.Cu") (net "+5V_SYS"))
 (segment (start 50.5 89) (end 50.5 95.09) (width 0.24) (layer "F.Cu") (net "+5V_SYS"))
 (segment (start 50 84.5) (end 50 85.5875) (width 0.35) (layer "F.Cu") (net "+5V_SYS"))
 (segment (start 58 84.5) (end 50 84.5) (width 0.35) (layer "F.Cu") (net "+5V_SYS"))
 (via (at 58 18.16) (size 0.8) (drill 0.4) (layers "F.Cu" "B.Cu") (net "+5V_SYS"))
 (via (at 58 36) (size 0.8) (drill 0.4) (layers "F.Cu" "B.Cu") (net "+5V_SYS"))
 (via (at 58 57) (size 0.8) (drill 0.4) (layers "F.Cu" "B.Cu") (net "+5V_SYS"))
 (via (at 58 84.5) (size 0.8) (drill 0.4) (layers "F.Cu" "B.Cu") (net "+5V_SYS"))
 (segment (start 50 119) (end 58 119) (width 0.9) (layer "B.Cu") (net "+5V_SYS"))
 (segment (start 58 119) (end 58 18.16) (width 0.9) (layer "B.Cu") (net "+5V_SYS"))
 (segment (start 46.9125 50) (end 52 50) (width 0.28) (layer "F.Cu") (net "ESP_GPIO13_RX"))
 (segment (start 52 50) (end 54.0875 50) (width 0.28) (layer "F.Cu") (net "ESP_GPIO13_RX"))
 (via (at 52 50) (size 0.8) (drill 0.4) (layers "F.Cu" "B.Cu") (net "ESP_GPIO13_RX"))
 (segment (start 52 15.62) (end 42 15.62) (width 0.28) (layer "B.Cu") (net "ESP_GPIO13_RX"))
 (segment (start 52 50) (end 52 15.62) (width 0.28) (layer "B.Cu") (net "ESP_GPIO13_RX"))
 (segment (start 50 43) (end 50 45) (width 0.28) (layer "F.Cu") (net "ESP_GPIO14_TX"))
 (segment (start 50 45) (end 46.9125 45) (width 0.28) (layer "F.Cu") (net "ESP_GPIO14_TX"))
 (via (at 50 43) (size 0.8) (drill 0.4) (layers "F.Cu" "B.Cu") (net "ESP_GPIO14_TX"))
 (segment (start 39.5 43) (end 50 43) (width 0.28) (layer "B.Cu") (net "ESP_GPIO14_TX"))
 (segment (start 42 20.7) (end 39.5 20.7) (width 0.28) (layer "B.Cu") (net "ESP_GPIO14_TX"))
 (segment (start 39.5 20.7) (end 39.5 43) (width 0.28) (layer "B.Cu") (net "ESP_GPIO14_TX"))
 (segment (start 61 20.7) (end 61 28) (width 0.28) (layer "F.Cu") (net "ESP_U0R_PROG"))
 (segment (start 64.86 20.7) (end 61 20.7) (width 0.28) (layer "F.Cu") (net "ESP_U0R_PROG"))
 (segment (start 61 28) (end 46.08 28) (width 0.28) (layer "F.Cu") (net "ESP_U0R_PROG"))
 (segment (start 46.08 28) (end 46.08 34) (width 0.28) (layer "F.Cu") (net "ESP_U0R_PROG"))
 (segment (start 64.86 23.24) (end 63.5 23.24) (width 0.28) (layer "F.Cu") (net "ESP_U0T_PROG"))
 (segment (start 63.5 31.5) (end 48.62 31.5) (width 0.28) (layer "F.Cu") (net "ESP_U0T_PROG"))
 (segment (start 48.62 31.5) (end 48.62 34) (width 0.28) (layer "F.Cu") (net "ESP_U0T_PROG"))
 (segment (start 63.5 23.24) (end 63.5 31.5) (width 0.28) (layer "F.Cu") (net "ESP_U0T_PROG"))
 (segment (start 60.5 39) (end 61 39) (width 0.28) (layer "B.Cu") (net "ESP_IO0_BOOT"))
 (segment (start 60.5 13.08) (end 60.5 39) (width 0.28) (layer "B.Cu") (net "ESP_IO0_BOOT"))
 (segment (start 64.86 13.08) (end 60.5 13.08) (width 0.28) (layer "B.Cu") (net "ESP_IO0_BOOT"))
 (segment (start 41.3 45) (end 45.0875 45) (width 0.28) (layer "F.Cu") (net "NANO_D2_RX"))
 (segment (start 33.4 72) (end 41.3 72) (width 0.28) (layer "F.Cu") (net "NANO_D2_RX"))
 (via (at 33.4 72) (size 0.8) (drill 0.4) (layers "F.Cu" "B.Cu") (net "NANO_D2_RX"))
 (via (at 41.3 45) (size 0.8) (drill 0.4) (layers "F.Cu" "B.Cu") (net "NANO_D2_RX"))
 (via (at 41.3 72) (size 0.8) (drill 0.4) (layers "F.Cu" "B.Cu") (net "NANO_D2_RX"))
 (segment (start 41.3 72) (end 41.3 45) (width 0.28) (layer "B.Cu") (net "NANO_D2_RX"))
 (segment (start 32.4 75.24) (end 33.4 72) (width 0.28) (layer "B.Cu") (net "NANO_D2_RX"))
 (segment (start 38.75 50) (end 45.0875 50) (width 0.28) (layer "F.Cu") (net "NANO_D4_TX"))
 (via (at 38.75 50) (size 0.8) (drill 0.4) (layers "F.Cu" "B.Cu") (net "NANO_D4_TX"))
 (segment (start 28.32 80) (end 38.75 80) (width 0.28) (layer "B.Cu") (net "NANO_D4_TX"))
 (segment (start 27.32 75.24) (end 28.32 80) (width 0.28) (layer "B.Cu") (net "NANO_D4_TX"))
 (segment (start 38.75 80) (end 38.75 50) (width 0.28) (layer "B.Cu") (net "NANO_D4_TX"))
 (segment (start 55 82) (end 61.0875 82) (width 0.24) (layer "F.Cu") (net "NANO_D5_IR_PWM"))
 (via (at 55 82) (size 0.8) (drill 0.4) (layers "F.Cu" "B.Cu") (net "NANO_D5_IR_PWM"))
 (segment (start 24.78 82) (end 55 82) (width 0.28) (layer "B.Cu") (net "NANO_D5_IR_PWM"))
 (segment (start 24.78 75.24) (end 24.78 82) (width 0.28) (layer "B.Cu") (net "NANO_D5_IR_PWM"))
 (segment (start 36 84) (end 37.0875 82) (width 0.24) (layer "F.Cu") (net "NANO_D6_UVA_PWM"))
 (via (at 36 84) (size 0.8) (drill 0.4) (layers "F.Cu" "B.Cu") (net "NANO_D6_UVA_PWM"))
 (segment (start 22.24 75.24) (end 22.24 84) (width 0.28) (layer "B.Cu") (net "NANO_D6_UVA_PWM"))
 (segment (start 22.24 84) (end 36 84) (width 0.28) (layer "B.Cu") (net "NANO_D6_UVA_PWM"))
 (segment (start 48 86) (end 49.0875 80) (width 0.28) (layer "F.Cu") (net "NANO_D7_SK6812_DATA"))
 (via (at 48 86) (size 0.8) (drill 0.4) (layers "F.Cu" "B.Cu") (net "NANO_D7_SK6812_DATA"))
 (segment (start 19.7 86) (end 48 86) (width 0.28) (layer "B.Cu") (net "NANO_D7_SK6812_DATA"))
 (segment (start 19.7 75.24) (end 19.7 86) (width 0.28) (layer "B.Cu") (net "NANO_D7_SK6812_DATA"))
 (segment (start 66.8 91.95) (end 63.9375 91.95) (width 0.24) (layer "F.Cu") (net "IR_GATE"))
 (segment (start 66.8 86.2) (end 66.8 91.95) (width 0.24) (layer "F.Cu") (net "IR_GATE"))
 (segment (start 62.9125 82) (end 63 86.2) (width 0.24) (layer "F.Cu") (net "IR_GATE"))
 (segment (start 62.9125 85) (end 63 86.2) (width 0.24) (layer "F.Cu") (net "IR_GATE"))
 (segment (start 63 86.2) (end 66.8 86.2) (width 0.24) (layer "F.Cu") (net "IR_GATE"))
 (segment (start 45.06 86.2) (end 45.0625 90.05) (width 0.24) (layer "F.Cu") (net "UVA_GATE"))
 (segment (start 40 86.2) (end 45.06 86.2) (width 0.24) (layer "F.Cu") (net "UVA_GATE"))
 (segment (start 38.9125 82) (end 40 86.2) (width 0.24) (layer "F.Cu") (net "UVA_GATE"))
 (segment (start 38.9125 85) (end 40 86.2) (width 0.24) (layer "F.Cu") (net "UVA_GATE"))
 (segment (start 62.0625 91) (end 57.5 91) (width 0.24) (layer "F.Cu") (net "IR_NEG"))
 (segment (start 57.5 91) (end 57.5 95.09) (width 0.24) (layer "F.Cu") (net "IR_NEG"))
 (segment (start 48.5 91) (end 48.5 95.09) (width 0.24) (layer "F.Cu") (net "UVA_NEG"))
 (segment (start 46.9375 91) (end 48.5 91) (width 0.24) (layer "F.Cu") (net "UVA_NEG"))
 (segment (start 56.5 88) (end 56.5 95.09) (width 0.24) (layer "F.Cu") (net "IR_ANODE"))
 (segment (start 58 87.4125) (end 56.5 88) (width 0.24) (layer "F.Cu") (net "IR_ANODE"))
 (segment (start 50 87.4125) (end 49.5 89.5) (width 0.24) (layer "F.Cu") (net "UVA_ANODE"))
 (segment (start 49.5 89.5) (end 49.5 95.09) (width 0.24) (layer "F.Cu") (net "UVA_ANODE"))
 (segment (start 50.9125 80) (end 52 80) (width 0.2) (layer "F.Cu") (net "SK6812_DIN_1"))
 (segment (start 54.5 93.6) (end 54.5 95.09) (width 0.2) (layer "F.Cu") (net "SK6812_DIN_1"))
 (via (at 54.5 93.6) (size 0.8) (drill 0.4) (layers "F.Cu" "B.Cu") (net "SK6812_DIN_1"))
 (via (at 52 80) (size 0.8) (drill 0.4) (layers "F.Cu" "B.Cu") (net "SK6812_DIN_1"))
 (segment (start 56.5 80) (end 56.5 86) (width 0.2) (layer "B.Cu") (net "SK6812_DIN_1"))
 (segment (start 54.5 86) (end 54.5 93.6) (width 0.2) (layer "B.Cu") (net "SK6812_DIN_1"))
 (segment (start 56.5 86) (end 54.5 86) (width 0.2) (layer "B.Cu") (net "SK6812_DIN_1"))
 (segment (start 52 80) (end 56.5 80) (width 0.2) (layer "B.Cu") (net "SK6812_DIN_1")))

